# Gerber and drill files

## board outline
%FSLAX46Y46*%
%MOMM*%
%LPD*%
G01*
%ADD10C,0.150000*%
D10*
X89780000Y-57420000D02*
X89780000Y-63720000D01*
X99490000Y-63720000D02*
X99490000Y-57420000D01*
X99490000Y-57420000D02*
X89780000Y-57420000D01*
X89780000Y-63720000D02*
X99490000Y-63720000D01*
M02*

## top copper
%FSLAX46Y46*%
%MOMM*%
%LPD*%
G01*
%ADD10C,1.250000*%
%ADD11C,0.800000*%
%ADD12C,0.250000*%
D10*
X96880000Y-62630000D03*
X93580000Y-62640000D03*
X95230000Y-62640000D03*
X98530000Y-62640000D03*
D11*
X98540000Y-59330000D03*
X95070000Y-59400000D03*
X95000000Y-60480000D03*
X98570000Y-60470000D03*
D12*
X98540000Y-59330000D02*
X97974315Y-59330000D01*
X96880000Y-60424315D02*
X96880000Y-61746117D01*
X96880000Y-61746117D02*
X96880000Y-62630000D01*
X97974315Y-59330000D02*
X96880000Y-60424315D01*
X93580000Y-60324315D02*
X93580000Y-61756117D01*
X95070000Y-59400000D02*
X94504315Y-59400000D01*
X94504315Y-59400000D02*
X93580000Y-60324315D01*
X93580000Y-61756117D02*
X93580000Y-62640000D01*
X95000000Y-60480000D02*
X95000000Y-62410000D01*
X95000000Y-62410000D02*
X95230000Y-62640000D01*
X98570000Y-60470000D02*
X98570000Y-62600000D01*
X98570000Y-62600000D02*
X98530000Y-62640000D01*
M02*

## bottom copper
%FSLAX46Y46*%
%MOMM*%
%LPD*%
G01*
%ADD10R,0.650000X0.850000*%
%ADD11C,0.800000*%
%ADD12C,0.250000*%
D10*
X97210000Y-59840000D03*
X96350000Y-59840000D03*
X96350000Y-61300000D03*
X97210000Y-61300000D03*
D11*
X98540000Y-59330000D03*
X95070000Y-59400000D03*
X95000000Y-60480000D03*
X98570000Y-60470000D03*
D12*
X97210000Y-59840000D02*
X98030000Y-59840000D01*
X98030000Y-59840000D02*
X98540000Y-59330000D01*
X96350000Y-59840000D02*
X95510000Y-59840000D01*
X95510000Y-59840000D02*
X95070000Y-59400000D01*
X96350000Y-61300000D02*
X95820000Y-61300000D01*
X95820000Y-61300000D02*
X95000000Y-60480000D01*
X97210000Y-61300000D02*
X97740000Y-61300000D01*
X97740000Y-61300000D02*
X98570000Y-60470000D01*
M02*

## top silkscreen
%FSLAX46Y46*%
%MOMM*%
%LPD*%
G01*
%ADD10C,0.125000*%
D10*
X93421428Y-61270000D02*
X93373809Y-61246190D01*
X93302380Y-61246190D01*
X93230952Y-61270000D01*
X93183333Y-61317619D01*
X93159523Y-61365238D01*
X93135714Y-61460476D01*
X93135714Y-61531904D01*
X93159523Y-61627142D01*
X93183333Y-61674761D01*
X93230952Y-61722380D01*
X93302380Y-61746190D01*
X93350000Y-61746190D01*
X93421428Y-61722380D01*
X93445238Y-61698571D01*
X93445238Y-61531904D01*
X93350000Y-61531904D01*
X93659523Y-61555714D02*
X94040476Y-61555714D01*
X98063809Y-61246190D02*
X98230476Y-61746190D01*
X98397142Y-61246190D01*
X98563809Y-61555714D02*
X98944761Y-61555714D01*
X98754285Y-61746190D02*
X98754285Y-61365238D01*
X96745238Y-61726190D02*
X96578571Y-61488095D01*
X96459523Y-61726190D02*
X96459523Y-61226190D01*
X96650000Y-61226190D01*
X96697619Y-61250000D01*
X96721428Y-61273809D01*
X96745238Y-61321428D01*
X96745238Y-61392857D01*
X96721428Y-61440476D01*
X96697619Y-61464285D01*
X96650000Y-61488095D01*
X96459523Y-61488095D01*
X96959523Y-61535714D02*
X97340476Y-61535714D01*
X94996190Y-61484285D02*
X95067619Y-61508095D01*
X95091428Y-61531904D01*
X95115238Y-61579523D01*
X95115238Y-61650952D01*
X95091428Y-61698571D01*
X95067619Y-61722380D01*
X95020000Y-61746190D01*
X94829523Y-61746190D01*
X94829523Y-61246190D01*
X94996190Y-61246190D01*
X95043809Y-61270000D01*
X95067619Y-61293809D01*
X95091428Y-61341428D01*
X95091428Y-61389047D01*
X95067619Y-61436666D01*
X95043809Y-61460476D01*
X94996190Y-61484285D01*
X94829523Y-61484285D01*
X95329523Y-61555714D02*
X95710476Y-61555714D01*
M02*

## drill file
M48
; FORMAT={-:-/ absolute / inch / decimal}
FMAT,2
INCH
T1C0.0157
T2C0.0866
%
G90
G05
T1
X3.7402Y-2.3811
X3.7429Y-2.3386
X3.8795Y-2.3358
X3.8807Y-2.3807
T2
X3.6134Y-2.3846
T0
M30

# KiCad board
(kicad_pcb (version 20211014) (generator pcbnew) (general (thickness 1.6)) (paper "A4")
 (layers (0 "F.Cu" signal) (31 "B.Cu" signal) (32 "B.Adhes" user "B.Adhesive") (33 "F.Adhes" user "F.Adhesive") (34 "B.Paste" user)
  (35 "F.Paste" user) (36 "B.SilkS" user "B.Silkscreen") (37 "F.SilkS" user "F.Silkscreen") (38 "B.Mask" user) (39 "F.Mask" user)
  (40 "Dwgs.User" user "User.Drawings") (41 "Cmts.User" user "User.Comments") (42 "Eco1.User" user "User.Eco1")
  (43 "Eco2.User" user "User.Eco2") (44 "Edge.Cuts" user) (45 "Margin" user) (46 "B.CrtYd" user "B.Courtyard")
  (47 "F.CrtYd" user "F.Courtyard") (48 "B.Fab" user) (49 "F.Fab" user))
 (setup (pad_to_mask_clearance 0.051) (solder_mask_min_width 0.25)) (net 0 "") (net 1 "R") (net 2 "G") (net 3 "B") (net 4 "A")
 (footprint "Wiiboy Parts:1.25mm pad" (layer "F.Cu") (at 96.88 62.63)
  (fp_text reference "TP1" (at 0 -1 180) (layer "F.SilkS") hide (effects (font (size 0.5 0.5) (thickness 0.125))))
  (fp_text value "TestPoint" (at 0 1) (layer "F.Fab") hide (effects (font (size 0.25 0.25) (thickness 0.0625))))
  (pad "1" smd circle locked (at 0 0) (size 1.25 1.25) (layers "F.Cu" "F.Paste" "F.Mask") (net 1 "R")))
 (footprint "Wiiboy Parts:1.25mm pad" (layer "F.Cu") (at 93.58 62.64)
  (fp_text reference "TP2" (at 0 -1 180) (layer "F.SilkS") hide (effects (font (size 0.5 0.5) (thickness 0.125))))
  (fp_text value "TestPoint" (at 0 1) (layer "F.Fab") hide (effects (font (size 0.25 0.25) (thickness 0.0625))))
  (pad "1" smd circle locked (at 0 0) (size 1.25 1.25) (layers "F.Cu" "F.Paste" "F.Mask") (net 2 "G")))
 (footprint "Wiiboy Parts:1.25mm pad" (layer "F.Cu") (at 95.23 62.64)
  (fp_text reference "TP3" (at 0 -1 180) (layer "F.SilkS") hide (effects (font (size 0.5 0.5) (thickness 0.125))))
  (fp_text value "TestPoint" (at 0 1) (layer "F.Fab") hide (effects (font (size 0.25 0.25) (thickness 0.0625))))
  (pad "1" smd circle locked (at 0 0) (size 1.25 1.25) (layers "F.Cu" "F.Paste" "F.Mask") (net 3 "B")))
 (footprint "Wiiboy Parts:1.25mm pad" (layer "F.Cu") (at 98.53 62.64)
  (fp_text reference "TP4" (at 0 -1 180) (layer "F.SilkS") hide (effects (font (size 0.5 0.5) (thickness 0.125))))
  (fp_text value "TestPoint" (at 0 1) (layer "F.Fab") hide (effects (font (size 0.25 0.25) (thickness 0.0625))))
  (pad "1" smd circle locked (at 0 0) (size 1.25 1.25) (layers "F.Cu" "F.Paste" "F.Mask") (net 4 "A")))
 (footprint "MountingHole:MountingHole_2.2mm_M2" (layer "F.Cu") (at 91.78 60.57)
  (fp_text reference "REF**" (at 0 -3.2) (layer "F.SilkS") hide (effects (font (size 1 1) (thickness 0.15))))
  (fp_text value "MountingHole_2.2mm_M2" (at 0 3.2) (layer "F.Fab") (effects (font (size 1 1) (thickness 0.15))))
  (pad "" np_thru_hole circle locked (at 0 0) (size 2.2 2.2) (drill 2.2) (layers *.Cu *.Mask)))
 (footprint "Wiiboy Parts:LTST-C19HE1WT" (layer "B.Cu") (at 96.78 60.57 180)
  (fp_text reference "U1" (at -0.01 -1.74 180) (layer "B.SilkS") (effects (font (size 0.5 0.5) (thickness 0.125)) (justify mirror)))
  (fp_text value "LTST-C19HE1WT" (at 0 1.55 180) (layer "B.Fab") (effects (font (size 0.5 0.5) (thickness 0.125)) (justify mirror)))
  (pad "1" smd rect locked (at -0.43 0.73 180) (size 0.65 0.85) (layers "B.Cu" "B.Paste" "B.Mask") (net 1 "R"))
  (pad "2" smd rect locked (at 0.43 0.73 180) (size 0.65 0.85) (layers "B.Cu" "B.Paste" "B.Mask") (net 2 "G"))
  (pad "3" smd rect locked (at 0.43 -0.73 180) (size 0.65 0.85) (layers "B.Cu" "B.Paste" "B.Mask") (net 3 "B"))
  (pad "4" smd rect locked (at -0.43 -0.73 180) (size 0.65 0.85) (layers "B.Cu" "B.Paste" "B.Mask") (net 4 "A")))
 (gr_line (start 89.78 57.42) (end 89.78 63.72) (layer "Edge.Cuts") (width 0.15))
 (gr_line (start 99.49 63.72) (end 99.49 57.42) (layer "Edge.Cuts") (width 0.15))
 (gr_line (start 99.49 57.42) (end 89.78 57.42) (layer "Edge.Cuts") (width 0.15))
 (gr_line (start 89.78 63.72) (end 99.49 63.72) (layer "Edge.Cuts") (width 0.15))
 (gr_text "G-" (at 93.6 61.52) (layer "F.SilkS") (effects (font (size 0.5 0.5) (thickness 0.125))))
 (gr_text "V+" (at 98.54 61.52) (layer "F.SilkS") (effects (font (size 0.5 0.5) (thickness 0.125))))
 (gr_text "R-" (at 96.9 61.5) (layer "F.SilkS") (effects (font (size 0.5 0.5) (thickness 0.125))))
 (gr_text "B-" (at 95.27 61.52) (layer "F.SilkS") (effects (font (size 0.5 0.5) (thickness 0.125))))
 (segment (start 98.54 59.33) (end 97.974315 59.33) (width 0.25) (layer "F.Cu") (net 1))
 (segment (start 96.88 60.424315) (end 96.88 61.746117) (width 0.25) (layer "F.Cu") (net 1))
 (segment (start 96.88 61.746117) (end 96.88 62.63) (width 0.25) (layer "F.Cu") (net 1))
 (segment (start 97.974315 59.33) (end 96.88 60.424315) (width 0.25) (layer "F.Cu") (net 1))
 (via (at 98.54 59.33) (size 0.8) (drill 0.4) (layers "F.Cu" "B.Cu") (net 1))
 (segment (start 97.21 59.84) (end 98.03 59.84) (width 0.25) (layer "B.Cu") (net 1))
 (segment (start 98.03 59.84) (end 98.54 59.33) (width 0.25) (layer "B.Cu") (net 1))
 (segment (start 93.58 60.324315) (end 93.58 61.756117) (width 0.25) (layer "F.Cu") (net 2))
 (segment (start 95.07 59.4) (end 94.504315 59.4) (width 0.25) (layer "F.Cu") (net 2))
 (segment (start 94.504315 59.4) (end 93.58 60.324315) (width 0.25) (layer "F.Cu") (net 2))
 (segment (start 93.58 61.756117) (end 93.58 62.64) (width 0.25) (layer "F.Cu") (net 2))
 (via (at 95.07 59.4) (size 0.8) (drill 0.4) (layers "F.Cu" "B.Cu") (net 2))
 (segment (start 96.35 59.84) (end 95.51 59.84) (width 0.25) (layer "B.Cu") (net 2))
 (segment (start 95.51 59.84) (end 95.07 59.4) (width 0.25) (layer "B.Cu") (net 2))
 (segment (start 95 60.48) (end 95 62.41) (width 0.25) (layer "F.Cu") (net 3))
 (segment (start 95 62.41) (end 95.23 62.64) (width 0.25) (layer "F.Cu") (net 3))
 (via (at 95 60.48) (size 0.8) (drill 0.4) (layers "F.Cu" "B.Cu") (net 3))
 (segment (start 96.35 61.3) (end 95.82 61.3) (width 0.25) (layer "B.Cu") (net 3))
 (segment (start 95.82 61.3) (end 95 60.48) (width 0.25) (layer "B.Cu") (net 3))
 (segment (start 98.57 60.47) (end 98.57 62.6) (width 0.25) (layer "F.Cu") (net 4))
 (segment (start 98.57 62.6) (end 98.53 62.64) (width 0.25) (layer "F.Cu") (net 4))
 (via (at 98.57 60.47) (size 0.8) (drill 0.4) (layers "F.Cu" "B.Cu") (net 4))
 (segment (start 97.21 61.3) (end 97.74 61.3) (width 0.25) (layer "B.Cu") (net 4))
 (segment (start 97.74 61.3) (end 98.57 60.47) (width 0.25) (layer "B.Cu") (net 4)))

